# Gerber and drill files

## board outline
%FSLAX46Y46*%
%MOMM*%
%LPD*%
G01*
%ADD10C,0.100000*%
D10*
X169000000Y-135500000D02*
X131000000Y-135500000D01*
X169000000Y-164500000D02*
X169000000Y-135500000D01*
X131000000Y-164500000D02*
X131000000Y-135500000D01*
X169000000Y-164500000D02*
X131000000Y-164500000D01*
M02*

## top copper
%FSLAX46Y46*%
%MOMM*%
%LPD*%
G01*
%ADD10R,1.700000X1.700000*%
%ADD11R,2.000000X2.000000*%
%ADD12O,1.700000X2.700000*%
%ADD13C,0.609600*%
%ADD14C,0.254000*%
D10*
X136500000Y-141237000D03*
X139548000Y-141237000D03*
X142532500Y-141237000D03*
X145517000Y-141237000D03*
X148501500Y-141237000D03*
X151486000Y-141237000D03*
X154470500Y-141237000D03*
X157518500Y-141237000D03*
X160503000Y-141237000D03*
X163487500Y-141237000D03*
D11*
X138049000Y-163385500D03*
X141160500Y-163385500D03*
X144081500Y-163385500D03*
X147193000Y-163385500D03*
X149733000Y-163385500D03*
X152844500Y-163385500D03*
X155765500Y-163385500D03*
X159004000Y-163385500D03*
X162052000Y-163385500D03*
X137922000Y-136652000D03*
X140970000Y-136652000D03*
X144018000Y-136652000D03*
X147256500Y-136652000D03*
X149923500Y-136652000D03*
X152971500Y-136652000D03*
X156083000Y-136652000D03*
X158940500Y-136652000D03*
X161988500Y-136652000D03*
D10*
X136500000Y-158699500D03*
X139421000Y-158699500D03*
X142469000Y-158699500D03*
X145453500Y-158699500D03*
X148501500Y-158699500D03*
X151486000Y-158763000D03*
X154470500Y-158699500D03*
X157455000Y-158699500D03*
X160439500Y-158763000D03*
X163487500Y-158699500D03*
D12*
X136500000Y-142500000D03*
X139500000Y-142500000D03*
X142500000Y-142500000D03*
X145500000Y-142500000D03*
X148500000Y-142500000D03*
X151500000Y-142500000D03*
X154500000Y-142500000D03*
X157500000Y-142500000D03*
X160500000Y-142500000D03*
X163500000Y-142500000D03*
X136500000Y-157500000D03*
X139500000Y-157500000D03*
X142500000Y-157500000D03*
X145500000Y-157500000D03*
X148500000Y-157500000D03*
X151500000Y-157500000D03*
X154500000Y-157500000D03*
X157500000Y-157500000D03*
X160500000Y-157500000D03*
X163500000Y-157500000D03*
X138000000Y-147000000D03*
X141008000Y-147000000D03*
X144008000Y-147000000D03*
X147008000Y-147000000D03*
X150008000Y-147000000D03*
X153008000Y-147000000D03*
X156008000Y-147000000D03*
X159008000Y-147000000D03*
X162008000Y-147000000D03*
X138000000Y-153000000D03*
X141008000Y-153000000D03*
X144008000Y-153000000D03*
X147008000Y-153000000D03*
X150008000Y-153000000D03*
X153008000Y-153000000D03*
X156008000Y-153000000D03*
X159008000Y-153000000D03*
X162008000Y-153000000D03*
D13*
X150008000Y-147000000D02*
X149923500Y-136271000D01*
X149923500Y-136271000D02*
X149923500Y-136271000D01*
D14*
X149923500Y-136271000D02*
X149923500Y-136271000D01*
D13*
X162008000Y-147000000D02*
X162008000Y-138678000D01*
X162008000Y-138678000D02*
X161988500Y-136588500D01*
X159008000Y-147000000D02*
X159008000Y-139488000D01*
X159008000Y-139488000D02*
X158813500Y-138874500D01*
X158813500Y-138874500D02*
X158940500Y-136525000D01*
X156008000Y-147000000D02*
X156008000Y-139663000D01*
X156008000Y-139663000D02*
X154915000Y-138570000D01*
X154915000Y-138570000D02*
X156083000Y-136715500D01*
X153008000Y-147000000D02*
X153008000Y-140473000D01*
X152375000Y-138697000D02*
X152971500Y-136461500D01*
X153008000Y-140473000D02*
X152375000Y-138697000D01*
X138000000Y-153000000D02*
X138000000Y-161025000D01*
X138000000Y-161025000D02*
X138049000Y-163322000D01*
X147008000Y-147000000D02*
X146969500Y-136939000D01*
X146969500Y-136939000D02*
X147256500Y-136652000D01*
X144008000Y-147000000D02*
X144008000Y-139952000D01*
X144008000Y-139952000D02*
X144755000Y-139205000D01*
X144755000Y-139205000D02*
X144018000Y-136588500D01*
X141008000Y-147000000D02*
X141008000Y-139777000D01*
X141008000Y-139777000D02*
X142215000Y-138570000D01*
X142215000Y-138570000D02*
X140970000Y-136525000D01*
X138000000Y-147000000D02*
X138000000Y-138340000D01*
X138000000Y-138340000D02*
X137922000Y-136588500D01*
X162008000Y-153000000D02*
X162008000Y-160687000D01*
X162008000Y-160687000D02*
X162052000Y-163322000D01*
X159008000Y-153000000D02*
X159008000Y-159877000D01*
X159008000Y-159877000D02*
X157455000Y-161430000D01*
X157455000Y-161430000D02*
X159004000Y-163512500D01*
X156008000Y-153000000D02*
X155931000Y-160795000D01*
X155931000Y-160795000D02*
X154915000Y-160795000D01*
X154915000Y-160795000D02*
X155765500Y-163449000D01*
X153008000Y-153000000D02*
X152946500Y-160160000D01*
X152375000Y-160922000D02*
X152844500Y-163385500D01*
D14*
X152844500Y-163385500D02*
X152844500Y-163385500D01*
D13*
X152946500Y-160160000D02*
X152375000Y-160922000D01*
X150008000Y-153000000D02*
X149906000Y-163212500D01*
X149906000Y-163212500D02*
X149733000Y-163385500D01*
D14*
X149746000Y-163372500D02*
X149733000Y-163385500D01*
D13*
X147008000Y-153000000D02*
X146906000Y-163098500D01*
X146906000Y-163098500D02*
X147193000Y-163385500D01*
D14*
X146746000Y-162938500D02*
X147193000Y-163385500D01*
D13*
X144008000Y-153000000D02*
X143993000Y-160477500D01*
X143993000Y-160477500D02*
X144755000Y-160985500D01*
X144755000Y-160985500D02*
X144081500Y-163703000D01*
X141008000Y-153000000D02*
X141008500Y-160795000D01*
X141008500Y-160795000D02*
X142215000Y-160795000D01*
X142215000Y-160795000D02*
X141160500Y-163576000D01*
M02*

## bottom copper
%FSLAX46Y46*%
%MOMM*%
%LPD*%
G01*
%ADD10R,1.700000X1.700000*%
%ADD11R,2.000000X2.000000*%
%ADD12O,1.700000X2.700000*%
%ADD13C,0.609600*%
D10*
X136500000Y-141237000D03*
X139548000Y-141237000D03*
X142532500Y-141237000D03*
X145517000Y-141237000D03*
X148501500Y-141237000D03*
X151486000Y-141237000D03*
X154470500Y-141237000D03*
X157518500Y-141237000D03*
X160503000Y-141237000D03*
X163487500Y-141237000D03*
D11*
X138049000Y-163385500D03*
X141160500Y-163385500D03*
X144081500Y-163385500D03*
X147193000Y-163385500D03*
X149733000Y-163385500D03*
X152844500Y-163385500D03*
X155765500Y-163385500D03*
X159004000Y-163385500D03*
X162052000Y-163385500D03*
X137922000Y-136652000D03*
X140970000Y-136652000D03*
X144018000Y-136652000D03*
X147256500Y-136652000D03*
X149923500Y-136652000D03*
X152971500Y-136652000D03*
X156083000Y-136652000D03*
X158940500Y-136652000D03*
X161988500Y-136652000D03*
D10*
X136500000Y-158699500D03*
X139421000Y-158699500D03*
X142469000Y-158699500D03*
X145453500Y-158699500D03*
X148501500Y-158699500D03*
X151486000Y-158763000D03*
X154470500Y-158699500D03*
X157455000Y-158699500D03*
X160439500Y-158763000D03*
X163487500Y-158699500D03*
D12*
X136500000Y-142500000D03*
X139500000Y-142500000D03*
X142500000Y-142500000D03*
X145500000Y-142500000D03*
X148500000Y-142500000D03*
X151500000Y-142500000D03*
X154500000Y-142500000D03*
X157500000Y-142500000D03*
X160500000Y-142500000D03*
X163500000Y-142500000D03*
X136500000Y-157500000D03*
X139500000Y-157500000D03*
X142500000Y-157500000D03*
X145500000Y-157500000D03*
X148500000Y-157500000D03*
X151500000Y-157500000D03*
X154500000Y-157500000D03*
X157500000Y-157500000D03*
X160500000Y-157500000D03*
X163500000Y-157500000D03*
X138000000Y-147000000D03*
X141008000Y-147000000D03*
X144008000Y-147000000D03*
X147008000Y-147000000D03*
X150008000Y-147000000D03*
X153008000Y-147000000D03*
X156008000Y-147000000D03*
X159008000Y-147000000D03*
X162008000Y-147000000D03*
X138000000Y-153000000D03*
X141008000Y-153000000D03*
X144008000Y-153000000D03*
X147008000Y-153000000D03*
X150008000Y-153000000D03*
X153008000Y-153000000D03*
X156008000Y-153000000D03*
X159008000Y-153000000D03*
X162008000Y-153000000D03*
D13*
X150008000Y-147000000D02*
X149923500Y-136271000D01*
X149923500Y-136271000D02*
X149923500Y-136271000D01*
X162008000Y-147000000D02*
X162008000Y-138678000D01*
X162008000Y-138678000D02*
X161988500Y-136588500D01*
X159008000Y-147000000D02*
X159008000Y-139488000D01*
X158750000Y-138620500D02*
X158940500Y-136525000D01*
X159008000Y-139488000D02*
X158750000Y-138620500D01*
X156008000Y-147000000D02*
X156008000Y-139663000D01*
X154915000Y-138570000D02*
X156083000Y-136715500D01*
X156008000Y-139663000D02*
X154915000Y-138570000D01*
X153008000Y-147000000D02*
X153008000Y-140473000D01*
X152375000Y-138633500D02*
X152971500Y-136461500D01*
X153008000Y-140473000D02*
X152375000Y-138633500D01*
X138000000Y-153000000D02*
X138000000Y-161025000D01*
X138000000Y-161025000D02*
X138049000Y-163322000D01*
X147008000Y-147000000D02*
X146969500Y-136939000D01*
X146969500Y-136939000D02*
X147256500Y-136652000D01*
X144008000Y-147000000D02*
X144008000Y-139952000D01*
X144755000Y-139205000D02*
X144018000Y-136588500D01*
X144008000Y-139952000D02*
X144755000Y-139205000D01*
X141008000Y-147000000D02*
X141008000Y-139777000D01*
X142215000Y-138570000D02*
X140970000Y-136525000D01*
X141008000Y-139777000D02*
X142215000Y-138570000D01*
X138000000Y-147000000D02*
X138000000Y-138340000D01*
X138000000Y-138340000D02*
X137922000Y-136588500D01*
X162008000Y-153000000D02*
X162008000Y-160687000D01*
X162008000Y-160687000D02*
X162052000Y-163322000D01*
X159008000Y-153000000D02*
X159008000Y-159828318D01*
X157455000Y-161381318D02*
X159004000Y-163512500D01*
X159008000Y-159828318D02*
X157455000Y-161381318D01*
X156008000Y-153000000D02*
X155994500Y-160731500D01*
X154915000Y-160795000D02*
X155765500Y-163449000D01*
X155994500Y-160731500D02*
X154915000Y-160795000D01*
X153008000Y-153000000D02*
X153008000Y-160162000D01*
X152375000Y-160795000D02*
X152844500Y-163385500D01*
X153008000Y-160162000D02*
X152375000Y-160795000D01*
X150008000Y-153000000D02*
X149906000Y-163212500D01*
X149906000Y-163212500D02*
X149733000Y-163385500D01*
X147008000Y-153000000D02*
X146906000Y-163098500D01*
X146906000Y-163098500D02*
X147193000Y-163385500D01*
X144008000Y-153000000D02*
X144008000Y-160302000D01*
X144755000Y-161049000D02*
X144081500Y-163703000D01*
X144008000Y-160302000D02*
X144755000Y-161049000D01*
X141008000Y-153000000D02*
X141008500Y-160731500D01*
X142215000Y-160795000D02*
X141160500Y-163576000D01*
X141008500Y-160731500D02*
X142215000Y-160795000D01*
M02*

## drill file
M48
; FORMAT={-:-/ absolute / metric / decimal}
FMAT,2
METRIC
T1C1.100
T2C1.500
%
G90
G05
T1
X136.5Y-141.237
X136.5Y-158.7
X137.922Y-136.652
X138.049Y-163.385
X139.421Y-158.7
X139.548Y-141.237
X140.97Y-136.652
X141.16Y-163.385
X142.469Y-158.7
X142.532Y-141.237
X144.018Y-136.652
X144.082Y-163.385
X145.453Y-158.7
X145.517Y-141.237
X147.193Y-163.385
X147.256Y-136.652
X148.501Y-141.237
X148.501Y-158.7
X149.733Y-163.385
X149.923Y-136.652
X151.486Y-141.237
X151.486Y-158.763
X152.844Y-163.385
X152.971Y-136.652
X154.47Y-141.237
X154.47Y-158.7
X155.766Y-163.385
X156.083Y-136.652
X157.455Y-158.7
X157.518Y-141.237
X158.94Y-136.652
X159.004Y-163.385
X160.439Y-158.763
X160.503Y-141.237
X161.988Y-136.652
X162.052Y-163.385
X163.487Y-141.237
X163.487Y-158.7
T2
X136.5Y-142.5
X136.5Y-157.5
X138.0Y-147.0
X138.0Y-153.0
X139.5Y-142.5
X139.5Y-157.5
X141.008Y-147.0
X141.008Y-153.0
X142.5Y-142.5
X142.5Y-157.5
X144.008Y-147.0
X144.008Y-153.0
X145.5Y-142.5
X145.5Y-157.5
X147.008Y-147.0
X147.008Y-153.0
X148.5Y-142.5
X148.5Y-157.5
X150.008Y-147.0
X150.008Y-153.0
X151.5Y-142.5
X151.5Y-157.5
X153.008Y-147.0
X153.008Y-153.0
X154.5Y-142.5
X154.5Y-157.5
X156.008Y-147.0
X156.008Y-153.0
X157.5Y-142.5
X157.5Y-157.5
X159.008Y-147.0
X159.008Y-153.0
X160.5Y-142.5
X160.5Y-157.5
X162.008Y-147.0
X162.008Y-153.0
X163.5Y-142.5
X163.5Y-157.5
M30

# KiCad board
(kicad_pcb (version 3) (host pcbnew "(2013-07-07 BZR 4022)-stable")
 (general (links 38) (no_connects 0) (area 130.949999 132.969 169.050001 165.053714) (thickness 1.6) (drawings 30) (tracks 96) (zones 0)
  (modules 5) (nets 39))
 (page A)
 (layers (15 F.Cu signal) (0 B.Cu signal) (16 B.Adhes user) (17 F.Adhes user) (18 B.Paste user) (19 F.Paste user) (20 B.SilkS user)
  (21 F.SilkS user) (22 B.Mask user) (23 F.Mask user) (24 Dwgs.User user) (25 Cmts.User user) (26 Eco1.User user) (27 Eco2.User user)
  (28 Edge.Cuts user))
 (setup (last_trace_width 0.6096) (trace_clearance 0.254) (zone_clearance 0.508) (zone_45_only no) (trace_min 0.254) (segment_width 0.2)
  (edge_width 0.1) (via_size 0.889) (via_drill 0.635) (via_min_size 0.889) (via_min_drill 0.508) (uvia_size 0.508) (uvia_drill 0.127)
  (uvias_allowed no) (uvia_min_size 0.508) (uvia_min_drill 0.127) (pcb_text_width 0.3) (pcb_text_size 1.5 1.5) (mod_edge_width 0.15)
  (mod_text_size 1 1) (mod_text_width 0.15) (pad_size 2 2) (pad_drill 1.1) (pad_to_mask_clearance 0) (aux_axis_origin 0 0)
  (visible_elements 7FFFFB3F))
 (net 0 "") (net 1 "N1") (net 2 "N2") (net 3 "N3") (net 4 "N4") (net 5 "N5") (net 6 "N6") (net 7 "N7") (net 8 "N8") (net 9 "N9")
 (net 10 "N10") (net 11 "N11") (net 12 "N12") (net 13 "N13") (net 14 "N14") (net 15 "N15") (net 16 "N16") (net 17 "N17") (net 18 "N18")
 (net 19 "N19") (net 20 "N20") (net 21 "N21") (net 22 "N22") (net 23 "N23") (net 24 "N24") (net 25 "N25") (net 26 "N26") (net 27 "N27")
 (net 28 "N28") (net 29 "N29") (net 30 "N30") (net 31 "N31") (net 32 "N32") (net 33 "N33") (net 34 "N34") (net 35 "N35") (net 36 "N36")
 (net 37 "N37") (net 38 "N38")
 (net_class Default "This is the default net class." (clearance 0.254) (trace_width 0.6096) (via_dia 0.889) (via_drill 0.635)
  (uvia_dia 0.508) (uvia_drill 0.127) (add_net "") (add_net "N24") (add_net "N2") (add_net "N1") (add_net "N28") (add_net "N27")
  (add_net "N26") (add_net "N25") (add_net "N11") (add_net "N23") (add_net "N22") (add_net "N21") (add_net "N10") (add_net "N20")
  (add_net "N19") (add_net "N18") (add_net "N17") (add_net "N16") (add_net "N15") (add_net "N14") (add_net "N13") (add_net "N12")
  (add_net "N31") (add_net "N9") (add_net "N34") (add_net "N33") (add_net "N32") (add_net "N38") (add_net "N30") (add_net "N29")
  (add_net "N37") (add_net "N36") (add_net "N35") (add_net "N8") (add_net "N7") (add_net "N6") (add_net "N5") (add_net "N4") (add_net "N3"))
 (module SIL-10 (layer F.Cu) (at 149.708 141.237)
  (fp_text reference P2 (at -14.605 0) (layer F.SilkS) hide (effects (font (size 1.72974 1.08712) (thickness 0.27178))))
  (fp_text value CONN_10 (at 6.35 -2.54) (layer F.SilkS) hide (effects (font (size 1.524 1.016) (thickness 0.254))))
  (pad 1 thru_hole rect (at -13.208 0) (size 1.7 1.7) (drill 1.1) (layers *.Cu *.Mask F.SilkS) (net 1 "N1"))
  (pad 2 thru_hole rect (at -10.16 0) (size 1.7 1.7) (drill 1.1) (layers *.Cu *.Mask F.SilkS) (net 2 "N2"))
  (pad 3 thru_hole rect (at -7.1755 0) (size 1.7 1.7) (drill 1.1) (layers *.Cu *.Mask F.SilkS) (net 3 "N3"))
  (pad 4 thru_hole rect (at -4.191 0) (size 1.7 1.7) (drill 1.1) (layers *.Cu *.Mask F.SilkS) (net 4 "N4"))
  (pad 5 thru_hole rect (at -1.2065 0) (size 1.7 1.7) (drill 1.1) (layers *.Cu *.Mask F.SilkS) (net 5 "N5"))
  (pad 6 thru_hole rect (at 1.778 0) (size 1.7 1.7) (drill 1.1) (layers *.Cu *.Mask F.SilkS) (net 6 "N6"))
  (pad 7 thru_hole rect (at 4.7625 0) (size 1.7 1.7) (drill 1.1) (layers *.Cu *.Mask F.SilkS) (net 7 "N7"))
  (pad 8 thru_hole rect (at 7.8105 0) (size 1.7 1.7) (drill 1.1) (layers *.Cu *.Mask F.SilkS) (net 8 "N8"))
  (pad 9 thru_hole rect (at 10.795 0) (size 1.7 1.7) (drill 1.1) (layers *.Cu *.Mask F.SilkS) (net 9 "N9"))
  (pad 10 thru_hole rect (at 13.7795 0) (size 1.7 1.7) (drill 1.1) (layers *.Cu *.Mask F.SilkS) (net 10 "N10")))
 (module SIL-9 (layer F.Cu) (at 149.733 163.3855)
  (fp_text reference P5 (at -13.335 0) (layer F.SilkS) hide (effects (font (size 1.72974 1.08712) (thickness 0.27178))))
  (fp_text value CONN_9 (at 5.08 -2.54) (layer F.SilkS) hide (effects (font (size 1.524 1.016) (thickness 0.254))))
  (pad 1 thru_hole rect (at -11.684 0) (size 2 2) (drill 1.1) (layers *.Cu *.Mask F.SilkS) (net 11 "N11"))
  (pad 2 thru_hole rect (at -8.5725 0) (size 2 2) (drill 1.1) (layers *.Cu *.Mask F.SilkS) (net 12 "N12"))
  (pad 3 thru_hole rect (at -5.6515 0) (size 2 2) (drill 1.1) (layers *.Cu *.Mask F.SilkS) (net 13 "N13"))
  (pad 4 thru_hole rect (at -2.54 0) (size 2 2) (drill 1.1) (layers *.Cu *.Mask F.SilkS) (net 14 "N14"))
  (pad 5 thru_hole rect (at 0 0) (size 2 2) (drill 1.1) (layers *.Cu *.Mask F.SilkS) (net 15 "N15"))
  (pad 6 thru_hole rect (at 3.1115 0) (size 2 2) (drill 1.1) (layers *.Cu *.Mask F.SilkS) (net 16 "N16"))
  (pad 7 thru_hole rect (at 6.0325 0) (size 2 2) (drill 1.1) (layers *.Cu *.Mask F.SilkS) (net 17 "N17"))
  (pad 8 thru_hole rect (at 9.271 0) (size 2 2) (drill 1.1) (layers *.Cu *.Mask F.SilkS) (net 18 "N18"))
  (pad 9 thru_hole rect (at 12.319 0) (size 2 2) (drill 1.1) (layers *.Cu *.Mask F.SilkS) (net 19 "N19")))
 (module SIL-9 (layer F.Cu) (at 149.7965 136.652)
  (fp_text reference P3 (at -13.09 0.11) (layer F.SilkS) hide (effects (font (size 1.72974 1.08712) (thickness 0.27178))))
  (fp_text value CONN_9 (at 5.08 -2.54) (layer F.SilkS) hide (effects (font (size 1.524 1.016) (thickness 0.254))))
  (pad 1 thru_hole rect (at -11.8745 0) (size 2 2) (drill 1.1) (layers *.Cu *.Mask F.SilkS) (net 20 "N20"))
  (pad 2 thru_hole rect (at -8.8265 0) (size 2 2) (drill 1.1) (layers *.Cu *.Mask F.SilkS) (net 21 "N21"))
  (pad 3 thru_hole rect (at -5.7785 0) (size 2 2) (drill 1.1) (layers *.Cu *.Mask F.SilkS) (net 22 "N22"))
  (pad 4 thru_hole rect (at -2.54 0) (size 2 2) (drill 1.1) (layers *.Cu *.Mask F.SilkS) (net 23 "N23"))
  (pad 5 thru_hole rect (at 0.127 0) (size 2 2) (drill 1.1) (layers *.Cu *.Mask F.SilkS) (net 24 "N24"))
  (pad 6 thru_hole rect (at 3.175 0) (size 2 2) (drill 1.1) (layers *.Cu *.Mask F.SilkS) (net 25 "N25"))
  (pad 7 thru_hole rect (at 6.2865 0) (size 2 2) (drill 1.1) (layers *.Cu *.Mask F.SilkS) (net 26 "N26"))
  (pad 8 thru_hole rect (at 9.144 0) (size 2 2) (drill 1.1) (layers *.Cu *.Mask F.SilkS) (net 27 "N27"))
  (pad 9 thru_hole rect (at 12.192 0) (size 2 2) (drill 1.1) (layers *.Cu *.Mask F.SilkS) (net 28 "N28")))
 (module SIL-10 (layer F.Cu) (at 149.2635 158.6995)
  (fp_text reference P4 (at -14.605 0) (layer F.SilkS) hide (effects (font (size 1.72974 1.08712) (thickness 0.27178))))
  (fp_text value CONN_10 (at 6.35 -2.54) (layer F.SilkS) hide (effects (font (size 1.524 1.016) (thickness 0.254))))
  (pad 1 thru_hole rect (at -12.7635 0) (size 1.7 1.7) (drill 1.1) (layers *.Cu *.Mask F.SilkS) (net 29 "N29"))
  (pad 2 thru_hole rect (at -9.8425 0) (size 1.7 1.7) (drill 1.1) (layers *.Cu *.Mask F.SilkS) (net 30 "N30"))
  (pad 3 thru_hole rect (at -6.7945 0) (size 1.7 1.7) (drill 1.1) (layers *.Cu *.Mask F.SilkS) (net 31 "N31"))
  (pad 4 thru_hole rect (at -3.81 0) (size 1.7 1.7) (drill 1.1) (layers *.Cu *.Mask F.SilkS) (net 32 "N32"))
  (pad 5 thru_hole rect (at -0.762 0) (size 1.7 1.7) (drill 1.1) (layers *.Cu *.Mask F.SilkS) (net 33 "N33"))
  (pad 6 thru_hole rect (at 2.2225 0.0635) (size 1.7 1.7) (drill 1.1) (layers *.Cu *.Mask F.SilkS) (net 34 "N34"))
  (pad 7 thru_hole rect (at 5.207 0) (size 1.7 1.7) (drill 1.1) (layers *.Cu *.Mask F.SilkS) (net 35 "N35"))
  (pad 8 thru_hole rect (at 8.1915 0) (size 1.7 1.7) (drill 1.1) (layers *.Cu *.Mask F.SilkS) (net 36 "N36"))
  (pad 9 thru_hole rect (at 11.176 0.0635) (size 1.7 1.7) (drill 1.1) (layers *.Cu *.Mask F.SilkS) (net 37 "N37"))
  (pad 10 thru_hole rect (at 14.224 0) (size 1.7 1.7) (drill 1.1) (layers *.Cu *.Mask F.SilkS) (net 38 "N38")))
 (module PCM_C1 (layer F.Cu) (at 136.5 150)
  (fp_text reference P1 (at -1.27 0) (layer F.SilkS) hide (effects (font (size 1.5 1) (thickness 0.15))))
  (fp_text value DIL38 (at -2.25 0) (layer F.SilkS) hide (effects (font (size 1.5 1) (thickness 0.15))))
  (pad 1 thru_hole oval (at 0 -7.5) (size 1.7 2.7) (drill 1.5) (layers *.Cu *.Mask F.SilkS) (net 1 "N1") (zone_connect 2))
  (pad 2 thru_hole oval (at 3 -7.5) (size 1.7 2.7) (drill 1.5) (layers *.Cu *.Mask F.SilkS) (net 2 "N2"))
  (pad 3 thru_hole oval (at 6 -7.5) (size 1.7 2.7) (drill 1.5) (layers *.Cu *.Mask F.SilkS) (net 3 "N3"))
  (pad 4 thru_hole oval (at 9 -7.5) (size 1.7 2.7) (drill 1.5) (layers *.Cu *.Mask F.SilkS) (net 4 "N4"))
  (pad 5 thru_hole oval (at 12 -7.5) (size 1.7 2.7) (drill 1.5) (layers *.Cu *.Mask F.SilkS) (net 5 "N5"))
  (pad 6 thru_hole oval (at 15 -7.5) (size 1.7 2.7) (drill 1.5) (layers *.Cu *.Mask F.SilkS) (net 6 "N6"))
  (pad 7 thru_hole oval (at 18 -7.5) (size 1.7 2.7) (drill 1.5) (layers *.Cu *.Mask F.SilkS) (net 7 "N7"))
  (pad 8 thru_hole oval (at 21 -7.5) (size 1.7 2.7) (drill 1.5) (layers *.Cu *.Mask F.SilkS) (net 8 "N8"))
  (pad 9 thru_hole oval (at 24 -7.5) (size 1.7 2.7) (drill 1.5) (layers *.Cu *.Mask F.SilkS) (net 9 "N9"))
  (pad 10 thru_hole oval (at 27 -7.5) (size 1.7 2.7) (drill 1.5) (layers *.Cu *.Mask F.SilkS) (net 10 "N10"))
  (pad 29 thru_hole oval (at 0 7.5) (size 1.7 2.7) (drill 1.5) (layers *.Cu *.Mask F.SilkS) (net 29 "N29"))
  (pad 30 thru_hole oval (at 3 7.5) (size 1.7 2.7) (drill 1.5) (layers *.Cu *.Mask F.SilkS) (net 30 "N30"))
  (pad 31 thru_hole oval (at 6 7.5) (size 1.7 2.7) (drill 1.5) (layers *.Cu *.Mask F.SilkS) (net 31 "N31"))
  (pad 32 thru_hole oval (at 9 7.5) (size 1.7 2.7) (drill 1.5) (layers *.Cu *.Mask F.SilkS) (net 32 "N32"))
  (pad 33 thru_hole oval (at 12 7.5) (size 1.7 2.7) (drill 1.5) (layers *.Cu *.Mask F.SilkS) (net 33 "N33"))
  (pad 34 thru_hole oval (at 15 7.5) (size 1.7 2.7) (drill 1.5) (layers *.Cu *.Mask F.SilkS) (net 34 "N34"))
  (pad 35 thru_hole oval (at 18 7.5) (size 1.7 2.7) (drill 1.5) (layers *.Cu *.Mask F.SilkS) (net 35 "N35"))
  (pad 36 thru_hole oval (at 21 7.5) (size 1.7 2.7) (drill 1.5) (layers *.Cu *.Mask F.SilkS) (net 36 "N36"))
  (pad 37 thru_hole oval (at 24 7.5) (size 1.7 2.7) (drill 1.5) (layers *.Cu *.Mask F.SilkS) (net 37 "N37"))
  (pad 38 thru_hole oval (at 27 7.5) (size 1.7 2.7) (drill 1.5) (layers *.Cu *.Mask F.SilkS) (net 38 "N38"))
  (pad 11 thru_hole oval (at 1.5 -3) (size 1.7 2.7) (drill 1.5) (layers *.Cu *.Mask F.SilkS) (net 20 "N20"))
  (pad 12 thru_hole oval (at 4.508 -3) (size 1.7 2.7) (drill 1.5) (layers *.Cu *.Mask F.SilkS) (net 21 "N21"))
  (pad 13 thru_hole oval (at 7.508 -3) (size 1.7 2.7) (drill 1.5) (layers *.Cu *.Mask F.SilkS) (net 22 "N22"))
  (pad 14 thru_hole oval (at 10.508 -3) (size 1.7 2.7) (drill 1.5) (layers *.Cu *.Mask F.SilkS) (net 23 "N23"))
  (pad 15 thru_hole oval (at 13.508 -3) (size 1.7 2.7) (drill 1.5) (layers *.Cu *.Mask F.SilkS) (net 24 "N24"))
  (pad 16 thru_hole oval (at 16.508 -3) (size 1.7 2.7) (drill 1.5) (layers *.Cu *.Mask F.SilkS) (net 25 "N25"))
  (pad 17 thru_hole oval (at 19.508 -3) (size 1.7 2.7) (drill 1.5) (layers *.Cu *.Mask F.SilkS) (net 26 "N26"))
  (pad 18 thru_hole oval (at 22.508 -3) (size 1.7 2.7) (drill 1.5) (layers *.Cu *.Mask F.SilkS) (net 27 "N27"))
  (pad 19 thru_hole oval (at 25.508 -3) (size 1.7 2.7) (drill 1.5) (layers *.Cu *.Mask F.SilkS) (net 28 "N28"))
  (pad 20 thru_hole oval (at 1.5 3) (size 1.7 2.7) (drill 1.5) (layers *.Cu *.Mask F.SilkS) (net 11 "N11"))
  (pad 21 thru_hole oval (at 4.508 3) (size 1.7 2.7) (drill 1.5) (layers *.Cu *.Mask F.SilkS) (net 12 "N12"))
  (pad 22 thru_hole oval (at 7.508 3) (size 1.7 2.7) (drill 1.5) (layers *.Cu *.Mask F.SilkS) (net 13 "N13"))
  (pad 23 thru_hole oval (at 10.508 3) (size 1.7 2.7) (drill 1.5) (layers *.Cu *.Mask F.SilkS) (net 14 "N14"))
  (pad 24 thru_hole oval (at 13.508 3) (size 1.7 2.7) (drill 1.5) (layers *.Cu *.Mask F.SilkS) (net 15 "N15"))
  (pad 25 thru_hole oval (at 16.508 3) (size 1.7 2.7) (drill 1.5) (layers *.Cu *.Mask F.SilkS) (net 16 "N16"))
  (pad 26 thru_hole oval (at 19.508 3) (size 1.7 2.7) (drill 1.5) (layers *.Cu *.Mask F.SilkS) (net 17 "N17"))
  (pad 27 thru_hole oval (at 22.508 3) (size 1.7 2.7) (drill 1.5) (layers *.Cu *.Mask F.SilkS) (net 18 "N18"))
  (pad 28 thru_hole oval (at 25.508 3) (size 1.7 2.7) (drill 1.5) (layers *.Cu *.Mask F.SilkS) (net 19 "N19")))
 (gr_line (start 169 135.5) (end 131 135.5) (angle 90) (layer Edge.Cuts) (width 0.1))
 (gr_line (start 169 164.5) (end 169 135.5) (angle 90) (layer Edge.Cuts) (width 0.1))
 (gr_line (start 131 164.5) (end 131 135.5) (angle 90) (layer Edge.Cuts) (width 0.1))
 (gr_line (start 169 164.5) (end 131 164.5) (angle 90) (layer Edge.Cuts) (width 0.1))
 (segment (start 150.008 147) (end 149.9235 136.271) (width 0.6096) (layer F.Cu) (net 24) (status 20))
 (segment (start 149.9235 136.271) (end 149.9235 136.271) (width 0.6096) (layer F.Cu) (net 24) (status 30))
 (segment (start 150.008 147) (end 149.9235 136.271) (width 0.6096) (layer B.Cu) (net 24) (status 20))
 (segment (start 149.9235 136.271) (end 149.9235 136.271) (width 0.6096) (layer B.Cu) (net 24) (status 30))
 (segment (start 149.9235 136.271) (end 149.9235 136.271) (width 0.254) (layer F.Cu) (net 24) (status 30))
 (segment (start 162.008 147) (end 162.008 138.678) (width 0.6096) (layer F.Cu) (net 28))
 (segment (start 162.008 138.678) (end 161.9885 136.5885) (width 0.6096) (layer F.Cu) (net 28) (status 20))
 (segment (start 162.008 147) (end 162.008 138.678) (width 0.6096) (layer B.Cu) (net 28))
 (segment (start 162.008 138.678) (end 161.9885 136.5885) (width 0.6096) (layer B.Cu) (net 28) (status 20))
 (segment (start 159.008 147) (end 159.008 139.488) (width 0.6096) (layer F.Cu) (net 27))
 (segment (start 159.008 139.488) (end 158.8135 138.8745) (width 0.6096) (layer F.Cu) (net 27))
 (segment (start 158.8135 138.8745) (end 158.9405 136.525) (width 0.6096) (layer F.Cu) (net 27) (status 20))
 (segment (start 159.008 147) (end 159.008 139.488) (width 0.6096) (layer B.Cu) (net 27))
 (segment (start 158.75 138.6205) (end 158.9405 136.525) (width 0.6096) (layer B.Cu) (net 27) (status 20))
 (segment (start 159.008 139.488) (end 158.75 138.6205) (width 0.6096) (layer B.Cu) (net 27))
 (segment (start 156.008 147) (end 156.008 139.663) (width 0.6096) (layer F.Cu) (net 26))
 (segment (start 156.008 139.663) (end 154.915 138.57) (width 0.6096) (layer F.Cu) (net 26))
 (segment (start 154.915 138.57) (end 156.083 136.7155) (width 0.6096) (layer F.Cu) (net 26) (status 20))
 (segment (start 156.008 147) (end 156.008 139.663) (width 0.6096) (layer B.Cu) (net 26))
 (segment (start 154.915 138.57) (end 156.083 136.7155) (width 0.6096) (layer B.Cu) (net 26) (status 20))
 (segment (start 156.008 139.663) (end 154.915 138.57) (width 0.6096) (layer B.Cu) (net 26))
 (segment (start 153.008 147) (end 153.008 140.473) (width 0.6096) (layer F.Cu) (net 25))
 (segment (start 152.375 138.697) (end 152.9715 136.4615) (width 0.6096) (layer F.Cu) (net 25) (status 20))
 (segment (start 153.008 147) (end 153.008 140.473) (width 0.6096) (layer B.Cu) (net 25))
 (segment (start 152.375 138.6335) (end 152.9715 136.4615) (width 0.6096) (layer B.Cu) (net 25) (status 20))
 (segment (start 153.008 140.473) (end 152.375 138.697) (width 0.6096) (layer F.Cu) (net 25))
 (segment (start 153.008 140.473) (end 152.375 138.6335) (width 0.6096) (layer B.Cu) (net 25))
 (segment (start 138 153) (end 138 161.025) (width 0.6096) (layer F.Cu) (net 11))
 (segment (start 138 161.025) (end 138.049 163.322) (width 0.6096) (layer F.Cu) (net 11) (status 20))
 (segment (start 138 153) (end 138 161.025) (width 0.6096) (layer B.Cu) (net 11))
 (segment (start 138 161.025) (end 138.049 163.322) (width 0.6096) (layer B.Cu) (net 11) (status 20))
 (segment (start 147.008 147) (end 146.9695 136.939) (width 0.6096) (layer F.Cu) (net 23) (status 20))
 (segment (start 146.9695 136.939) (end 147.2565 136.652) (width 0.6096) (layer F.Cu) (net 23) (status 30))
 (segment (start 147.008 147) (end 146.9695 136.939) (width 0.6096) (layer B.Cu) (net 23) (status 20))
 (segment (start 146.9695 136.939) (end 147.2565 136.652) (width 0.6096) (layer B.Cu) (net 23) (status 30))
 (segment (start 144.008 147) (end 144.008 139.952) (width 0.6096) (layer F.Cu) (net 22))
 (segment (start 144.008 139.952) (end 144.755 139.205) (width 0.6096) (layer F.Cu) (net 22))
 (segment (start 144.755 139.205) (end 144.018 136.5885) (width 0.6096) (layer F.Cu) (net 22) (status 20))
 (segment (start 144.008 147) (end 144.008 139.952) (width 0.6096) (layer B.Cu) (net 22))
 (segment (start 144.755 139.205) (end 144.018 136.5885) (width 0.6096) (layer B.Cu) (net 22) (status 20))
 (segment (start 144.008 139.952) (end 144.755 139.205) (width 0.6096) (layer B.Cu) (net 22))
 (segment (start 141.008 147) (end 141.008 139.777) (width 0.6096) (layer F.Cu) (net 21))
 (segment (start 141.008 139.777) (end 142.215 138.57) (width 0.6096) (layer F.Cu) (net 21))
 (segment (start 142.215 138.57) (end 140.97 136.525) (width 0.6096) (layer F.Cu) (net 21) (status 20))
 (segment (start 141.008 147) (end 141.008 139.777) (width 0.6096) (layer B.Cu) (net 21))
 (segment (start 142.215 138.57) (end 140.97 136.525) (width 0.6096) (layer B.Cu) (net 21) (status 20))
 (segment (start 141.008 139.777) (end 142.215 138.57) (width 0.6096) (layer B.Cu) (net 21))
 (segment (start 138 147) (end 138 138.34) (width 0.6096) (layer F.Cu) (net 20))
 (segment (start 138 138.34) (end 137.922 136.5885) (width 0.6096) (layer F.Cu) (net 20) (status 20))
 (segment (start 138 147) (end 138 138.34) (width 0.6096) (layer B.Cu) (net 20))
 (segment (start 138 138.34) (end 137.922 136.5885) (width 0.6096) (layer B.Cu) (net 20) (status 20))
 (segment (start 162.008 153) (end 162.008 160.687) (width 0.6096) (layer F.Cu) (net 19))
 (segment (start 162.008 160.687) (end 162.052 163.322) (width 0.6096) (layer F.Cu) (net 19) (status 20))
 (segment (start 162.008 153) (end 162.008 160.687) (width 0.6096) (layer B.Cu) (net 19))
 (segment (start 162.008 160.687) (end 162.052 163.322) (width 0.6096) (layer B.Cu) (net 19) (status 20))
 (segment (start 159.008 153) (end 159.008 159.877) (width 0.6096) (layer F.Cu) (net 18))
 (segment (start 159.008 159.877) (end 157.455 161.43) (width 0.6096) (layer F.Cu) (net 18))
 (segment (start 157.455 161.43) (end 159.004 163.5125) (width 0.6096) (layer F.Cu) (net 18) (status 20))
 (segment (start 159.008 153) (end 159.008 159.828318) (width 0.6096) (layer B.Cu) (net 18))
 (segment (start 157.455 161.381318) (end 159.004 163.5125) (width 0.6096) (layer B.Cu) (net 18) (status 20))
 (segment (start 159.008 159.828318) (end 157.455 161.381318) (width 0.6096) (layer B.Cu) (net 18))
 (segment (start 156.008 153) (end 155.931 160.795) (width 0.6096) (layer F.Cu) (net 17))
 (segment (start 155.931 160.795) (end 154.915 160.795) (width 0.6096) (layer F.Cu) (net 17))
 (segment (start 154.915 160.795) (end 155.7655 163.449) (width 0.6096) (layer F.Cu) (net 17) (status 20))
 (segment (start 156.008 153) (end 155.9945 160.7315) (width 0.6096) (layer B.Cu) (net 17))
 (segment (start 154.915 160.795) (end 155.7655 163.449) (width 0.6096) (layer B.Cu) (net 17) (status 20))
 (segment (start 155.9945 160.7315) (end 154.915 160.795) (width 0.6096) (layer B.Cu) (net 17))
 (segment (start 153.008 153) (end 152.9465 160.16) (width 0.6096) (layer F.Cu) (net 16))
 (segment (start 152.375 160.922) (end 152.8445 163.3855) (width 0.6096) (layer F.Cu) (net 16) (status 20))
 (segment (start 153.008 153) (end 153.008 160.162) (width 0.6096) (layer B.Cu) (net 16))
 (segment (start 152.375 160.795) (end 152.8445 163.3855) (width 0.6096) (layer B.Cu) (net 16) (status 20))
 (segment (start 152.8445 163.3855) (end 152.8445 163.3855) (width 0.254) (layer F.Cu) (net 16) (status 30))
 (segment (start 152.9465 160.16) (end 152.375 160.922) (width 0.6096) (layer F.Cu) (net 16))
 (segment (start 153.008 160.162) (end 152.375 160.795) (width 0.6096) (layer B.Cu) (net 16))
 (segment (start 150.008 153) (end 149.906 163.2125) (width 0.6096) (layer F.Cu) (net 15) (status 20))
 (segment (start 149.906 163.2125) (end 149.733 163.3855) (width 0.6096) (layer F.Cu) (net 15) (status 30))
 (segment (start 150.008 153) (end 149.906 163.2125) (width 0.6096) (layer B.Cu) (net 15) (status 20))
 (segment (start 149.906 163.2125) (end 149.733 163.3855) (width 0.6096) (layer B.Cu) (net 15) (status 30))
 (segment (start 149.746 163.3725) (end 149.733 163.3855) (width 0.254) (layer F.Cu) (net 15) (status 30))
 (segment (start 147.008 153) (end 146.906 163.0985) (width 0.6096) (layer F.Cu) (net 14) (status 20))
 (segment (start 146.906 163.0985) (end 147.193 163.3855) (width 0.6096) (layer F.Cu) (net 14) (status 30))
 (segment (start 147.008 153) (end 146.906 163.0985) (width 0.6096) (layer B.Cu) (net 14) (status 20))
 (segment (start 146.906 163.0985) (end 147.193 163.3855) (width 0.6096) (layer B.Cu) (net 14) (status 30))
 (segment (start 146.746 162.9385) (end 147.193 163.3855) (width 0.254) (layer F.Cu) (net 14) (status 30))
 (segment (start 144.008 153) (end 143.993 160.4775) (width 0.6096) (layer F.Cu) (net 13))
 (segment (start 143.993 160.4775) (end 144.755 160.9855) (width 0.6096) (layer F.Cu) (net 13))
 (segment (start 144.755 160.9855) (end 144.0815 163.703) (width 0.6096) (layer F.Cu) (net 13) (status 20))
 (segment (start 144.008 153) (end 144.008 160.302) (width 0.6096) (layer B.Cu) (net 13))
 (segment (start 144.755 161.049) (end 144.0815 163.703) (width 0.6096) (layer B.Cu) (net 13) (status 20))
 (segment (start 144.008 160.302) (end 144.755 161.049) (width 0.6096) (layer B.Cu) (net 13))
 (segment (start 141.008 153) (end 141.0085 160.795) (width 0.6096) (layer F.Cu) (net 12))
 (segment (start 141.0085 160.795) (end 142.215 160.795) (width 0.6096) (layer F.Cu) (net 12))
 (segment (start 142.215 160.795) (end 141.1605 163.576) (width 0.6096) (layer F.Cu) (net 12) (status 20))
 (segment (start 141.008 153) (end 141.0085 160.7315) (width 0.6096) (layer B.Cu) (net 12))
 (segment (start 142.215 160.795) (end 141.1605 163.576) (width 0.6096) (layer B.Cu) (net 12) (status 20))
 (segment (start 141.0085 160.7315) (end 142.215 160.795) (width 0.6096) (layer B.Cu) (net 12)))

